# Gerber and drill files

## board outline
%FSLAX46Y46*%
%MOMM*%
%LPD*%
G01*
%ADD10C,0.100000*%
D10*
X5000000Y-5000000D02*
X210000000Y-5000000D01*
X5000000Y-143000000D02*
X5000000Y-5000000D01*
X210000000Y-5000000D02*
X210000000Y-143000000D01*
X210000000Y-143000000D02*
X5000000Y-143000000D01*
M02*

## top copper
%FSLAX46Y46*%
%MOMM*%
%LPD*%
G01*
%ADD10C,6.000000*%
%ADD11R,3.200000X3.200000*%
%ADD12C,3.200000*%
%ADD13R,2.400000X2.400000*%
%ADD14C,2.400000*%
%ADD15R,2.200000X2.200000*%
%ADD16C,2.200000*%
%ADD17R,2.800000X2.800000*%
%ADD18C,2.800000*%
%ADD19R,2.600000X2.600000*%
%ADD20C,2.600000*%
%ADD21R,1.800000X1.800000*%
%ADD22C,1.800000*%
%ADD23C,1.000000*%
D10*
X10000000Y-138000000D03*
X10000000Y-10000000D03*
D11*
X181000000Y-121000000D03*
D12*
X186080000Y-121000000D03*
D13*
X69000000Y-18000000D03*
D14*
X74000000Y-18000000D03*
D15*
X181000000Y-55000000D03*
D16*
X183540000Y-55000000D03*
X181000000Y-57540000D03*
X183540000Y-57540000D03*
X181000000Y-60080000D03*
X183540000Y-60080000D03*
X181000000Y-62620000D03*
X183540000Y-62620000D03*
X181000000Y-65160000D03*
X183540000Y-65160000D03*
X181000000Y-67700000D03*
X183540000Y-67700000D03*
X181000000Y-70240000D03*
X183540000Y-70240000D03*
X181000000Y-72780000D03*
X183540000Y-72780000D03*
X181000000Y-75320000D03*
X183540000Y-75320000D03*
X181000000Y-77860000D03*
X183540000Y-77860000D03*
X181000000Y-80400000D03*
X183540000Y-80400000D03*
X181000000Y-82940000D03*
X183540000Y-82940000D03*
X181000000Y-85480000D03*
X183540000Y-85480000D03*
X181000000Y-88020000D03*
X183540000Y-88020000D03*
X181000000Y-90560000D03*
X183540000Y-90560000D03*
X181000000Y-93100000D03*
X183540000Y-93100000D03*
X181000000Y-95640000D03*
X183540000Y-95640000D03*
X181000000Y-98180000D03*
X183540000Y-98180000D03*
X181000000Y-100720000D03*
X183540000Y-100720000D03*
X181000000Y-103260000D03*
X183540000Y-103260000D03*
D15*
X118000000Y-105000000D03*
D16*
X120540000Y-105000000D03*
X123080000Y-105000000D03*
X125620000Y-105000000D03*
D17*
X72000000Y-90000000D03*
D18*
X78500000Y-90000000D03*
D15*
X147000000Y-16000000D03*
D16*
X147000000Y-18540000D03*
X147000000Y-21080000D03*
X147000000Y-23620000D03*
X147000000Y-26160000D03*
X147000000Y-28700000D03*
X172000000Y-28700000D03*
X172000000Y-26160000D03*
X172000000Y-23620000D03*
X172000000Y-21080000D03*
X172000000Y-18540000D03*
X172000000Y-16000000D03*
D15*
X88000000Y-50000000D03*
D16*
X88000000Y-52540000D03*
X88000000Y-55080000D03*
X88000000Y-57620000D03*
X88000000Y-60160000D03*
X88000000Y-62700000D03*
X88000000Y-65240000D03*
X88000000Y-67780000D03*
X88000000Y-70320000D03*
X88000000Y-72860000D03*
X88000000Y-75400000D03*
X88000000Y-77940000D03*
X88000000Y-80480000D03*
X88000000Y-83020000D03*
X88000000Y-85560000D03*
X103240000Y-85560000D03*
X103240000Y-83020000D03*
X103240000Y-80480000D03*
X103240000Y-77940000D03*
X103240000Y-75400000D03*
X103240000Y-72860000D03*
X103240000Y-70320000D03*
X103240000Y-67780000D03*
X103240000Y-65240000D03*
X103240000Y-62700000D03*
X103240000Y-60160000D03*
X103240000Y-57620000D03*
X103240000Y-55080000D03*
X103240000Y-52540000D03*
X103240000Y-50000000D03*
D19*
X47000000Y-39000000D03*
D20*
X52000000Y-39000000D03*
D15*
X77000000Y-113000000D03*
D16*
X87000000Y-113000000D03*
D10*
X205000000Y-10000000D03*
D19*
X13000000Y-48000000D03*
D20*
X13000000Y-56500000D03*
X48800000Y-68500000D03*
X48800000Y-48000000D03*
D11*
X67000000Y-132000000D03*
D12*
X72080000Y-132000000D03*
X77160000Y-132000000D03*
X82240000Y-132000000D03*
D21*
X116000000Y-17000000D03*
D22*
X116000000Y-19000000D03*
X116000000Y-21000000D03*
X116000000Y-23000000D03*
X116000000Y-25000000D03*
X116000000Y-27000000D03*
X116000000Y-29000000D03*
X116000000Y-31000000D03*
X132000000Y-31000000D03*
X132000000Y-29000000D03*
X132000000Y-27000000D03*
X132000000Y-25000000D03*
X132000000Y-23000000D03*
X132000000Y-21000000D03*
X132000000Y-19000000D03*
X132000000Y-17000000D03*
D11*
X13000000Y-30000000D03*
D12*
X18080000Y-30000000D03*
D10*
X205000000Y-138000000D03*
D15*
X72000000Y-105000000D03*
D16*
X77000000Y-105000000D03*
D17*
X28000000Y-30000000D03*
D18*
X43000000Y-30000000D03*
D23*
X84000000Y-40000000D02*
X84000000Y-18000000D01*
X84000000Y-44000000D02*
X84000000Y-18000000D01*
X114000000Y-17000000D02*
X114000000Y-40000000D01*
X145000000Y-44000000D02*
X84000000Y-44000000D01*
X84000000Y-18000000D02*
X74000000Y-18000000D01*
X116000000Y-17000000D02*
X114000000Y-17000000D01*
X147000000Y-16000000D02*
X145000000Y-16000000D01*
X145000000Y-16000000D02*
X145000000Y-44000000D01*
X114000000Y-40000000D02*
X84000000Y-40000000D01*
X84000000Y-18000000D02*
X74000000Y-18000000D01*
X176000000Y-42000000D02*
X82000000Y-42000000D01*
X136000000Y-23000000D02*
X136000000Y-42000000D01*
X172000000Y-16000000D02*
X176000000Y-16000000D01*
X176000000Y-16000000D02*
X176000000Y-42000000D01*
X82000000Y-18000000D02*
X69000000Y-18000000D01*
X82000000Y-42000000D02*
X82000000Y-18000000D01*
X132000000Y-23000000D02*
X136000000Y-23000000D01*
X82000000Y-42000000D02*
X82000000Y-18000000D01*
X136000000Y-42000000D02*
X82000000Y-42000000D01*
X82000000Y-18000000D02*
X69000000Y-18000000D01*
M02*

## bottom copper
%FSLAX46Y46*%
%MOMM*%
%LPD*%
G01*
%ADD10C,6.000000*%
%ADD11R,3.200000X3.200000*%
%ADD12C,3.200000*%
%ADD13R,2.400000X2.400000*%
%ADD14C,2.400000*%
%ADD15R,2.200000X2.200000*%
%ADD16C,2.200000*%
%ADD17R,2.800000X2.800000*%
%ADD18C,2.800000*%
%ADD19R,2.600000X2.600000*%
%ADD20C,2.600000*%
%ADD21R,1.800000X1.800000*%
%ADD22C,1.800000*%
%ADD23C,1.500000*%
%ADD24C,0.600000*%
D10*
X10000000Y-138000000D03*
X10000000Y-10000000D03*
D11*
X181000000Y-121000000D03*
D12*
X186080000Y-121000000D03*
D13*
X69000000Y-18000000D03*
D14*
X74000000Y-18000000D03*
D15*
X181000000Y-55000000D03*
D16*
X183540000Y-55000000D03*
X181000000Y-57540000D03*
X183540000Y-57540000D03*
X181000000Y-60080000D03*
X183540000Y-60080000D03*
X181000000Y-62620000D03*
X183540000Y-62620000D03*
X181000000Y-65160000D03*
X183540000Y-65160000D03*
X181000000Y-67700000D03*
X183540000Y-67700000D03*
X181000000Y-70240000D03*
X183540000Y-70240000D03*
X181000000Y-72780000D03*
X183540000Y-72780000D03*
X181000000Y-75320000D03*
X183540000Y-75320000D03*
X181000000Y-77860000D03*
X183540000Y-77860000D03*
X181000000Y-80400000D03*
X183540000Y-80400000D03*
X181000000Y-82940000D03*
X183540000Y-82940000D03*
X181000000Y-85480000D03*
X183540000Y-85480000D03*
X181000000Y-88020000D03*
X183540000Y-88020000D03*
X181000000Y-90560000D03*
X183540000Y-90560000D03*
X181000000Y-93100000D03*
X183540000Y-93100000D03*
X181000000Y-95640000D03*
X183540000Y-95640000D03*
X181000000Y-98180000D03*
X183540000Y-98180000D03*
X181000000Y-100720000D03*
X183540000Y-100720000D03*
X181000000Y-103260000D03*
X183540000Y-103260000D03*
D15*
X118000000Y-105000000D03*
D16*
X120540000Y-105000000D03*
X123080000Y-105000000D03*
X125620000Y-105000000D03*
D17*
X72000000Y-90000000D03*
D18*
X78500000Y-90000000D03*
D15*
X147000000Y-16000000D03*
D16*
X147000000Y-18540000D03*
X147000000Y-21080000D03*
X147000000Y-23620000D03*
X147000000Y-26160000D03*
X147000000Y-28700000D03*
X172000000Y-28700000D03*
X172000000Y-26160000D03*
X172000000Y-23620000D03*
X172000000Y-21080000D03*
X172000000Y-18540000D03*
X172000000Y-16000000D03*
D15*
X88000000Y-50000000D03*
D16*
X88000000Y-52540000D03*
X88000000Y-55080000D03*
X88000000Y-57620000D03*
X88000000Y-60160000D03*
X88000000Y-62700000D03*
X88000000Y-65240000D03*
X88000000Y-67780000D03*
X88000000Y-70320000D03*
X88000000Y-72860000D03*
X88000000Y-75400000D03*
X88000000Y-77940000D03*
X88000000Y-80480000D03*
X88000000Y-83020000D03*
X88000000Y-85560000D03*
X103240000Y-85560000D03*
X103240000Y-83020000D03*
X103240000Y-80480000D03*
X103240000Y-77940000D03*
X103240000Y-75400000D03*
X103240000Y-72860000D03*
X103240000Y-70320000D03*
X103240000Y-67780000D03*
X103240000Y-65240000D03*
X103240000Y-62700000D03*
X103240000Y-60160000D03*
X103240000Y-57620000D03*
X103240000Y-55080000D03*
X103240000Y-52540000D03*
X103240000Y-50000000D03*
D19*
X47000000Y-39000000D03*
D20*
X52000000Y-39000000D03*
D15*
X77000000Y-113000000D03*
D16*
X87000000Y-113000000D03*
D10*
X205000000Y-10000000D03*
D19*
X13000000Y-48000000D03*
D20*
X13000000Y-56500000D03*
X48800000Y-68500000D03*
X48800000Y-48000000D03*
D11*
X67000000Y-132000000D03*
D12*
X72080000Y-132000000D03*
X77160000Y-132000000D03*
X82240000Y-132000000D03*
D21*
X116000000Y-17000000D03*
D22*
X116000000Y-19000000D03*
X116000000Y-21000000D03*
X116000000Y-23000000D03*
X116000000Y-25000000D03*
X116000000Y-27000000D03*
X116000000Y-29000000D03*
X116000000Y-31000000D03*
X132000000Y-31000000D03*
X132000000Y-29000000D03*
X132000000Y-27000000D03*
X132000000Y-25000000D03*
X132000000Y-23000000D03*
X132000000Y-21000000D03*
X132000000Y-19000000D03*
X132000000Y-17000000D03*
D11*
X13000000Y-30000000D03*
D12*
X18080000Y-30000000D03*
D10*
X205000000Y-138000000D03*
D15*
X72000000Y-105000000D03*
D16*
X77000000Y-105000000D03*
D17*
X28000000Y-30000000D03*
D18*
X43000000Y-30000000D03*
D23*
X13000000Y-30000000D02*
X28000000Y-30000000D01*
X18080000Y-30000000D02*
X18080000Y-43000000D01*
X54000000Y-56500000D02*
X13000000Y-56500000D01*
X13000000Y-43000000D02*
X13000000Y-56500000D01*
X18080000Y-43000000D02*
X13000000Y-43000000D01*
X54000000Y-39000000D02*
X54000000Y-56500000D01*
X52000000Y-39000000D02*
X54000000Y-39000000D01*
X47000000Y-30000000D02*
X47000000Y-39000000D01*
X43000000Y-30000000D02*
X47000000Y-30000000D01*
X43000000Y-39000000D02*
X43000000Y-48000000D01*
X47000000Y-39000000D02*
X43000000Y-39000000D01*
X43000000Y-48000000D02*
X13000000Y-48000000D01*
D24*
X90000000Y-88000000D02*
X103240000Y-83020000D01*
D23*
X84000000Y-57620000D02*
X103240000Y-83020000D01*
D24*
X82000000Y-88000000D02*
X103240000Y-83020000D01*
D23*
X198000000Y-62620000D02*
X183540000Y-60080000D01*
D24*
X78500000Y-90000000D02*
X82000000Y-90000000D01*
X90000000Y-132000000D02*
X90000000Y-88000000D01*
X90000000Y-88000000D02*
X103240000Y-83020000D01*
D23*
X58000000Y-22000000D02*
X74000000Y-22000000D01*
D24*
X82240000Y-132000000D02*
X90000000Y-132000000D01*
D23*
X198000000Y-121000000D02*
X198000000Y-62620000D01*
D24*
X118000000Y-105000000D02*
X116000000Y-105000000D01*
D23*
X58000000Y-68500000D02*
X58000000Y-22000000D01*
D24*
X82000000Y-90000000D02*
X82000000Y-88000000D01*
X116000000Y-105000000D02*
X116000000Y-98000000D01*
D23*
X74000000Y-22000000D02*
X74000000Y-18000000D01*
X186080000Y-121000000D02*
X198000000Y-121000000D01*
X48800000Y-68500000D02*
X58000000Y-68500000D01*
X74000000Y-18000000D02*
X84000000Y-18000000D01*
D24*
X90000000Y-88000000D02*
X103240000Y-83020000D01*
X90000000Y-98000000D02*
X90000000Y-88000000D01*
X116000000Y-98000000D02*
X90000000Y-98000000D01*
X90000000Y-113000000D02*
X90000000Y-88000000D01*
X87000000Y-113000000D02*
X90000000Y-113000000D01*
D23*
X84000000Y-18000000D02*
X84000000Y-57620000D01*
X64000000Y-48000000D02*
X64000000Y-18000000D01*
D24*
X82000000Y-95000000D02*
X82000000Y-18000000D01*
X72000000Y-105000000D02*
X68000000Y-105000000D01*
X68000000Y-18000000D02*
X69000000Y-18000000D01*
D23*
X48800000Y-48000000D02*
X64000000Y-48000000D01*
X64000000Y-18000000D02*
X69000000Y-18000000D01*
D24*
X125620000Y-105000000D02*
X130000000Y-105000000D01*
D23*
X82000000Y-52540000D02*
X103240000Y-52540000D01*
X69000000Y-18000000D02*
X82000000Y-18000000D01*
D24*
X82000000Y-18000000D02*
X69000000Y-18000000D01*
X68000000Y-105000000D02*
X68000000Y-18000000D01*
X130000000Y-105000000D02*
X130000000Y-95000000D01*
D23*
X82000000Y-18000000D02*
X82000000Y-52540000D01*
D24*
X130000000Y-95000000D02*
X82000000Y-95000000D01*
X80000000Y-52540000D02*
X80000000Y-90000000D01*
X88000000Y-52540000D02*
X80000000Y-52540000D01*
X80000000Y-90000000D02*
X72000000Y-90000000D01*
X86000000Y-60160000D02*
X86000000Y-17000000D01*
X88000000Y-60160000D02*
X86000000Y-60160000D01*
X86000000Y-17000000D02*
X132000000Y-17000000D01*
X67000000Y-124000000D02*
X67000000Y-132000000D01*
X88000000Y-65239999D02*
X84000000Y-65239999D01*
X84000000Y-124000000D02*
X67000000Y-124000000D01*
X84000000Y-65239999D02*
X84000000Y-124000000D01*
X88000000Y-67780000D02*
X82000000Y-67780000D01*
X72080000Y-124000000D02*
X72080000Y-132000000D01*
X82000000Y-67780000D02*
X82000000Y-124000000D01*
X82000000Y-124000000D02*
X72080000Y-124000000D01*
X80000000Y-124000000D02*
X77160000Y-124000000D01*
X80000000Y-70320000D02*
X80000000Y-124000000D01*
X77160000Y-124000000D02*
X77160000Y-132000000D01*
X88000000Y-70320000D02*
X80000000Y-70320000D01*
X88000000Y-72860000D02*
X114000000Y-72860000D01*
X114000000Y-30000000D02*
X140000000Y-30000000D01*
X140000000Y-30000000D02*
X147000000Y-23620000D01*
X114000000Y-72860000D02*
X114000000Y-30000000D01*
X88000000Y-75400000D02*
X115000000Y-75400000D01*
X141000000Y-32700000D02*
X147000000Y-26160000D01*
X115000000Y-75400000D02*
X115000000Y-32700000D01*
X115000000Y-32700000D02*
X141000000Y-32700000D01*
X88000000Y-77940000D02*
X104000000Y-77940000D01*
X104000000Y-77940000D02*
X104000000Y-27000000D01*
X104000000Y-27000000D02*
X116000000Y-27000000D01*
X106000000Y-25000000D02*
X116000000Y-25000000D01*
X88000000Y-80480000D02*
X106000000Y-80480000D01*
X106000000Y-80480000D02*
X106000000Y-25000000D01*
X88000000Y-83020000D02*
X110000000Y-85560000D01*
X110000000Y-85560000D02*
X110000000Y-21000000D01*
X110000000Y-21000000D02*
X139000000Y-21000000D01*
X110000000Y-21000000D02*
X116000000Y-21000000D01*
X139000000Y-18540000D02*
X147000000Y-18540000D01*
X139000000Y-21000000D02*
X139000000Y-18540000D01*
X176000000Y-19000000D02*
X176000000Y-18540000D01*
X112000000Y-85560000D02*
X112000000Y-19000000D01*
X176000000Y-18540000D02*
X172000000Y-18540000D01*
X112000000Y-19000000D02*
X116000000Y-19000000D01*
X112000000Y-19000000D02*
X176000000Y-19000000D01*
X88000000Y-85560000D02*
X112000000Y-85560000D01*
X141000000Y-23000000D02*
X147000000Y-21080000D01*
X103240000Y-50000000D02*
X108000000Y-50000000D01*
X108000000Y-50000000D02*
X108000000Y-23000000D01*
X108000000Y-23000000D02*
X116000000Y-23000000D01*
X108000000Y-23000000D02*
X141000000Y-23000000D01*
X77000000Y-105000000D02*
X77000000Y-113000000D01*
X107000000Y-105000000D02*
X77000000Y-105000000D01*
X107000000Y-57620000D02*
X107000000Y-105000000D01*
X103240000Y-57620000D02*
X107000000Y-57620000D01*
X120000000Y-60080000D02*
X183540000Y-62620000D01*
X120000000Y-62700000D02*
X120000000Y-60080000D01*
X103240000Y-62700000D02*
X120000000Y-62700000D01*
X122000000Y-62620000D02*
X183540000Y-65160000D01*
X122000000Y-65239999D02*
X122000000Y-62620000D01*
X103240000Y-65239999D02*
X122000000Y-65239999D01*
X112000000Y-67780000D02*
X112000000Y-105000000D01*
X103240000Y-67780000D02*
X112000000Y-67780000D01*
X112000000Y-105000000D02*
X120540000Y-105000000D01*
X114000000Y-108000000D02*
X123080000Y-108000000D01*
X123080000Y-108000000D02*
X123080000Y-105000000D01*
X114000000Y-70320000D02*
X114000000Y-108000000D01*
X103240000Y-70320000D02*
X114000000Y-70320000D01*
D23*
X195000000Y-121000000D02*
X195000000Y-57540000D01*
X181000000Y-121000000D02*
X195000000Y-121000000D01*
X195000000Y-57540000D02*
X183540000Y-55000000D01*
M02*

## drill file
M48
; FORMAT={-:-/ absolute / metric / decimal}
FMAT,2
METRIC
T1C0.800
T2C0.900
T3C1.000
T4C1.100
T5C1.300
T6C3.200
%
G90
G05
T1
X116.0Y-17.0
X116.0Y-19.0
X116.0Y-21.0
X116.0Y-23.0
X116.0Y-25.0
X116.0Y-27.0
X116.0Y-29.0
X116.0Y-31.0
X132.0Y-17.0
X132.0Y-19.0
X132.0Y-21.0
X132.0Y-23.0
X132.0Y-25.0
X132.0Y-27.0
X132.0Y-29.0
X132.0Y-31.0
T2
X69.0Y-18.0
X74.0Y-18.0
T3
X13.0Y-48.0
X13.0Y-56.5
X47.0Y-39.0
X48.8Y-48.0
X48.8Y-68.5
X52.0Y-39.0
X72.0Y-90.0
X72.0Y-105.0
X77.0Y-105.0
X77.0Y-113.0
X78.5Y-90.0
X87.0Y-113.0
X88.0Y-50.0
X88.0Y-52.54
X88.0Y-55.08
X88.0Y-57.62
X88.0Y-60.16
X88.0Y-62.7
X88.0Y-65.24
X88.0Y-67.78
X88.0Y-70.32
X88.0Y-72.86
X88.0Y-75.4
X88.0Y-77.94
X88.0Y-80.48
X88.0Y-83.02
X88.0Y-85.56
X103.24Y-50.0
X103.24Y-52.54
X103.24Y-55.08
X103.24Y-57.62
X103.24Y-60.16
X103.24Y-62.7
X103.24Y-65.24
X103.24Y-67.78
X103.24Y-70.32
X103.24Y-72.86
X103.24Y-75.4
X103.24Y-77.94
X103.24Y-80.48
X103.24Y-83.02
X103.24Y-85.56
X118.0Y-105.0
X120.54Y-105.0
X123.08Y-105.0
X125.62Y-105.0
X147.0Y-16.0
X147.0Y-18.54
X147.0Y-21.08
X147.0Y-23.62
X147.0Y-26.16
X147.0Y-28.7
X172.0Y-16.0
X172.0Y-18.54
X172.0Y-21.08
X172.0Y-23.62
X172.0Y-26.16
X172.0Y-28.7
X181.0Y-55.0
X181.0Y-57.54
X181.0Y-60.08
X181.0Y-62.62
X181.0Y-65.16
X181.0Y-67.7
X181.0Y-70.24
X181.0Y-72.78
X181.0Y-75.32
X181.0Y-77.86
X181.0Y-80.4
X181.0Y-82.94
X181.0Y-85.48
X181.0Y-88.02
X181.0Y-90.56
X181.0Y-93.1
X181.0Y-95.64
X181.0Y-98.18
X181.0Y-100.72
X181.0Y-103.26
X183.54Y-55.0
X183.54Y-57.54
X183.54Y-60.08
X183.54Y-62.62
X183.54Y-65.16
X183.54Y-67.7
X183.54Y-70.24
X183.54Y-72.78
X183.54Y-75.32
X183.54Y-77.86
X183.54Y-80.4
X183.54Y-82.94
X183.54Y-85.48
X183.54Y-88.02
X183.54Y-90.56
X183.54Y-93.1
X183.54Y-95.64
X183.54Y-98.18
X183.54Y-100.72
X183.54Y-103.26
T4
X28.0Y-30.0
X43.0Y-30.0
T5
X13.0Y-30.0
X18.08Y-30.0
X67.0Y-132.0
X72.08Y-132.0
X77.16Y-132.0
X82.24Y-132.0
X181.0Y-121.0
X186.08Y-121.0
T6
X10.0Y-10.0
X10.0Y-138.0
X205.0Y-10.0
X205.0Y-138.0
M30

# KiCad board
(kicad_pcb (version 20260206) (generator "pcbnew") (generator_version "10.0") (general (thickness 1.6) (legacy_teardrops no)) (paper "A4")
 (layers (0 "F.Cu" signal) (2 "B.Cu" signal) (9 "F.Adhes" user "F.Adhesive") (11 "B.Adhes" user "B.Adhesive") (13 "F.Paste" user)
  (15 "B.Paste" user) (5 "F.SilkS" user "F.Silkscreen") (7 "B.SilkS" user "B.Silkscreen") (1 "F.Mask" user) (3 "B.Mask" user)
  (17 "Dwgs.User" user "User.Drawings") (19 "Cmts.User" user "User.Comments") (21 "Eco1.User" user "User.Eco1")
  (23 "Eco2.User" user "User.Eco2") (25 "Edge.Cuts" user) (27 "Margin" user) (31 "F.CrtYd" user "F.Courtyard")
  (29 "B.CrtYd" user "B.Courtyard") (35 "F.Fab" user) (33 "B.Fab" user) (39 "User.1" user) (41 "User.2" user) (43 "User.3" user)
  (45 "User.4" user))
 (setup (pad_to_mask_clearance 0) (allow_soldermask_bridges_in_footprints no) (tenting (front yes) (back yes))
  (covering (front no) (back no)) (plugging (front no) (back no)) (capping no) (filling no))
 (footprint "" (layer "F.Cu") (at 10 138)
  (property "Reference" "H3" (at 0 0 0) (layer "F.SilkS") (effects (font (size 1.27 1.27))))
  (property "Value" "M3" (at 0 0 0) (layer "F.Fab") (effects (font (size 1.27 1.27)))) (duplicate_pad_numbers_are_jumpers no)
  (pad "1" thru_hole circle (at 0 0) (size 6 6) (drill 3.2) (layers "*.Cu" "*.Mask") (remove_unused_layers no)))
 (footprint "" (layer "F.Cu") (at 10 10)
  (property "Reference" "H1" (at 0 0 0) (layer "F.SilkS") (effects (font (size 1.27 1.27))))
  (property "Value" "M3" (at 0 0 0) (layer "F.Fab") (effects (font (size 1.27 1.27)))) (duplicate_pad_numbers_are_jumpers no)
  (pad "1" thru_hole circle (at 0 0) (size 6 6) (drill 3.2) (layers "*.Cu" "*.Mask") (remove_unused_layers no)))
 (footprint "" (layer "F.Cu") (at 181 121)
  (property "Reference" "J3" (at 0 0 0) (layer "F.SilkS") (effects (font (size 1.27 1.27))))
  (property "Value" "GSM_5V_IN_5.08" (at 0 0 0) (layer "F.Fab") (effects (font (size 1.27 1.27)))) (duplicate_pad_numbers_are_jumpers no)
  (pad "1" thru_hole rect (at 0 0) (size 3.2 3.2) (drill 1.3) (layers "*.Cu" "*.Mask") (remove_unused_layers no) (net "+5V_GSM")
   (thermal_bridge_angle 45))
  (pad "2" thru_hole circle (at 5.08 0) (size 3.2 3.2) (drill 1.3) (layers "*.Cu" "*.Mask") (remove_unused_layers no) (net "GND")))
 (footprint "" (layer "F.Cu") (at 69 18)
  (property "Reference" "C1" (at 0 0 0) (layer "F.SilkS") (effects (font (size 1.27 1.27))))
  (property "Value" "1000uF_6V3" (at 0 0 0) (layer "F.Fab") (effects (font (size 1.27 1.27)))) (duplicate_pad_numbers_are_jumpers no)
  (pad "1" thru_hole rect (at 0 0) (size 2.4 2.4) (drill 0.9) (layers "*.Cu" "*.Mask") (remove_unused_layers no) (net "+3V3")
   (thermal_bridge_angle 45))
  (pad "2" thru_hole circle (at 5 0) (size 2.4 2.4) (drill 0.9) (layers "*.Cu" "*.Mask") (remove_unused_layers no) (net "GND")))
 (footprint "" (layer "F.Cu") (at 181 55)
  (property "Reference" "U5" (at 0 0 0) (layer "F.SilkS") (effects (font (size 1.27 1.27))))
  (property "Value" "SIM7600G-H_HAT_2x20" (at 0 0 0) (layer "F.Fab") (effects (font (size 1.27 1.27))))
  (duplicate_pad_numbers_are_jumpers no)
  (pad "1" thru_hole rect (at 0 0) (size 2.2 2.2) (drill 1) (layers "*.Cu" "*.Mask") (remove_unused_layers no) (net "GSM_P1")
   (thermal_bridge_angle 45))
  (pad "2" thru_hole circle (at 2.54 0) (size 2.2 2.2) (drill 1) (layers "*.Cu" "*.Mask") (remove_unused_layers no) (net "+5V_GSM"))
  (pad "3" thru_hole circle (at 0 2.54) (size 2.2 2.2) (drill 1) (layers "*.Cu" "*.Mask") (remove_unused_layers no) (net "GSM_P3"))
  (pad "4" thru_hole circle (at 2.54 2.54) (size 2.2 2.2) (drill 1) (layers "*.Cu" "*.Mask") (remove_unused_layers no) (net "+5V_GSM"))
  (pad "5" thru_hole circle (at 0 5.08) (size 2.2 2.2) (drill 1) (layers "*.Cu" "*.Mask") (remove_unused_layers no) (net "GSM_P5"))
  (pad "6" thru_hole circle (at 2.54 5.08) (size 2.2 2.2) (drill 1) (layers "*.Cu" "*.Mask") (remove_unused_layers no) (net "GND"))
  (pad "7" thru_hole circle (at 0 7.62) (size 2.2 2.2) (drill 1) (layers "*.Cu" "*.Mask") (remove_unused_layers no) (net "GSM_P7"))
  (pad "8" thru_hole circle (at 2.54 7.62) (size 2.2 2.2) (drill 1) (layers "*.Cu" "*.Mask") (remove_unused_layers no) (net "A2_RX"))
  (pad "9" thru_hole circle (at 0 10.16) (size 2.2 2.2) (drill 1) (layers "*.Cu" "*.Mask") (remove_unused_layers no) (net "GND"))
  (pad "10" thru_hole circle (at 2.54 10.16) (size 2.2 2.2) (drill 1) (layers "*.Cu" "*.Mask") (remove_unused_layers no) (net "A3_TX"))
  (pad "11" thru_hole circle (at 0 12.7) (size 2.2 2.2) (drill 1) (layers "*.Cu" "*.Mask") (remove_unused_layers no) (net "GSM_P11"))
  (pad "12" thru_hole circle (at 2.54 12.7) (size 2.2 2.2) (drill 1) (layers "*.Cu" "*.Mask") (remove_unused_layers no) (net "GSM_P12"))
  (pad "13" thru_hole circle (at 0 15.24) (size 2.2 2.2) (drill 1) (layers "*.Cu" "*.Mask") (remove_unused_layers no) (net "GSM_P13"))
  (pad "14" thru_hole circle (at 2.54 15.24) (size 2.2 2.2) (drill 1) (layers "*.Cu" "*.Mask") (remove_unused_layers no) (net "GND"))
  (pad "15" thru_hole circle (at 0 17.78) (size 2.2 2.2) (drill 1) (layers "*.Cu" "*.Mask") (remove_unused_layers no) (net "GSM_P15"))
  (pad "16" thru_hole circle (at 2.54 17.78) (size 2.2 2.2) (drill 1) (layers "*.Cu" "*.Mask") (remove_unused_layers no) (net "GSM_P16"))
  (pad "17" thru_hole circle (at 0 20.32) (size 2.2 2.2) (drill 1) (layers "*.Cu" "*.Mask") (remove_unused_layers no) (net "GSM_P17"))
  (pad "18" thru_hole circle (at 2.54 20.32) (size 2.2 2.2) (drill 1) (layers "*.Cu" "*.Mask") (remove_unused_layers no) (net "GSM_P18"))
  (pad "19" thru_hole circle (at 0 22.86) (size 2.2 2.2) (drill 1) (layers "*.Cu" "*.Mask") (remove_unused_layers no) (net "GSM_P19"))
  (pad "20" thru_hole circle (at 2.54 22.86) (size 2.2 2.2) (drill 1) (layers "*.Cu" "*.Mask") (remove_unused_layers no) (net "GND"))
  (pad "21" thru_hole circle (at 0 25.4) (size 2.2 2.2) (drill 1) (layers "*.Cu" "*.Mask") (remove_unused_layers no) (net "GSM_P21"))
  (pad "22" thru_hole circle (at 2.54 25.4) (size 2.2 2.2) (drill 1) (layers "*.Cu" "*.Mask") (remove_unused_layers no) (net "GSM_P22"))
  (pad "23" thru_hole circle (at 0 27.94) (size 2.2 2.2) (drill 1) (layers "*.Cu" "*.Mask") (remove_unused_layers no) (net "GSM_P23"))
  (pad "24" thru_hole circle (at 2.54 27.94) (size 2.2 2.2) (drill 1) (layers "*.Cu" "*.Mask") (remove_unused_layers no) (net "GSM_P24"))
  (pad "25" thru_hole circle (at 0 30.48) (size 2.2 2.2) (drill 1) (layers "*.Cu" "*.Mask") (remove_unused_layers no) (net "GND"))
  (pad "26" thru_hole circle (at 2.54 30.48) (size 2.2 2.2) (drill 1) (layers "*.Cu" "*.Mask") (remove_unused_layers no) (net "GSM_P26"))
  (pad "27" thru_hole circle (at 0 33.02) (size 2.2 2.2) (drill 1) (layers "*.Cu" "*.Mask") (remove_unused_layers no) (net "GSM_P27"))
  (pad "28" thru_hole circle (at 2.54 33.02) (size 2.2 2.2) (drill 1) (layers "*.Cu" "*.Mask") (remove_unused_layers no) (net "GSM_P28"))
  (pad "29" thru_hole circle (at 0 35.56) (size 2.2 2.2) (drill 1) (layers "*.Cu" "*.Mask") (remove_unused_layers no) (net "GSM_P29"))
  (pad "30" thru_hole circle (at 2.54 35.56) (size 2.2 2.2) (drill 1) (layers "*.Cu" "*.Mask") (remove_unused_layers no) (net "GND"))
  (pad "31" thru_hole circle (at 0 38.1) (size 2.2 2.2) (drill 1) (layers "*.Cu" "*.Mask") (remove_unused_layers no) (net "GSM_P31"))
  (pad "32" thru_hole circle (at 2.54 38.1) (size 2.2 2.2) (drill 1) (layers "*.Cu" "*.Mask") (remove_unused_layers no) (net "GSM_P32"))
  (pad "33" thru_hole circle (at 0 40.64) (size 2.2 2.2) (drill 1) (layers "*.Cu" "*.Mask") (remove_unused_layers no) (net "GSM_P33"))
  (pad "34" thru_hole circle (at 2.54 40.64) (size 2.2 2.2) (drill 1) (layers "*.Cu" "*.Mask") (remove_unused_layers no) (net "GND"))
  (pad "35" thru_hole circle (at 0 43.18) (size 2.2 2.2) (drill 1) (layers "*.Cu" "*.Mask") (remove_unused_layers no) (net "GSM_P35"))
  (pad "36" thru_hole circle (at 2.54 43.18) (size 2.2 2.2) (drill 1) (layers "*.Cu" "*.Mask") (remove_unused_layers no) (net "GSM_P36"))
  (pad "37" thru_hole circle (at 0 45.72) (size 2.2 2.2) (drill 1) (layers "*.Cu" "*.Mask") (remove_unused_layers no) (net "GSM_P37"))
  (pad "38" thru_hole circle (at 2.54 45.72) (size 2.2 2.2) (drill 1) (layers "*.Cu" "*.Mask") (remove_unused_layers no) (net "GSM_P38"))
  (pad "39" thru_hole circle (at 0 48.26) (size 2.2 2.2) (drill 1) (layers "*.Cu" "*.Mask") (remove_unused_layers no) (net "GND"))
  (pad "40" thru_hole circle (at 2.54 48.26) (size 2.2 2.2) (drill 1) (layers "*.Cu" "*.Mask") (remove_unused_layers no) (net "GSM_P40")))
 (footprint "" (layer "F.Cu") (at 118 105)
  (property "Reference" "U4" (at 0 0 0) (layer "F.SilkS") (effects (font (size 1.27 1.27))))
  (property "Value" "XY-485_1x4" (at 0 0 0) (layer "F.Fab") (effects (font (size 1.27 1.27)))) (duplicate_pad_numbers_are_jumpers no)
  (pad "1" thru_hole rect (at 0 0) (size 2.2 2.2) (drill 1) (layers "*.Cu" "*.Mask") (remove_unused_layers no) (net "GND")
   (thermal_bridge_angle 45))
  (pad "2" thru_hole circle (at 2.54 0) (size 2.2 2.2) (drill 1) (layers "*.Cu" "*.Mask") (remove_unused_layers no) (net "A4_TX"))
  (pad "3" thru_hole circle (at 5.08 0) (size 2.2 2.2) (drill 1) (layers "*.Cu" "*.Mask") (remove_unused_layers no) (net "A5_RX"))
  (pad "4" thru_hole circle (at 7.62 0) (size 2.2 2.2) (drill 1) (layers "*.Cu" "*.Mask") (remove_unused_layers no) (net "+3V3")))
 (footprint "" (layer "F.Cu") (at 72 90)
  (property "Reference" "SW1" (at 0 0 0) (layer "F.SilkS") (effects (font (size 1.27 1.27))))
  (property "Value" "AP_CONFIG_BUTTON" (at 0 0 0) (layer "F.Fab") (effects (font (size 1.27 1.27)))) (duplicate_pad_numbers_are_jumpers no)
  (pad "1" thru_hole rect (at 0 0) (size 2.8 2.8) (drill 1) (layers "*.Cu" "*.Mask") (remove_unused_layers no) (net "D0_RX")
   (thermal_bridge_angle 45))
  (pad "2" thru_hole circle (at 6.5 0) (size 2.8 2.8) (drill 1) (layers "*.Cu" "*.Mask") (remove_unused_layers no) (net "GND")))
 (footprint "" (layer "F.Cu") (at 147 16)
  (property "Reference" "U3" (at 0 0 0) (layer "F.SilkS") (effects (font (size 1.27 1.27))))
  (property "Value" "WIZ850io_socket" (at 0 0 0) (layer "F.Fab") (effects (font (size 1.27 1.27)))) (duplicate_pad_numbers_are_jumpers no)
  (pad "1" thru_hole rect (at 0 0) (size 2.2 2.2) (drill 1) (layers "*.Cu" "*.Mask") (remove_unused_layers no) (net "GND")
   (thermal_bridge_angle 45))
  (pad "2" thru_hole circle (at 0 2.54) (size 2.2 2.2) (drill 1) (layers "*.Cu" "*.Mask") (remove_unused_layers no) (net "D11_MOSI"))
  (pad "3" thru_hole circle (at 0 5.08) (size 2.2 2.2) (drill 1) (layers "*.Cu" "*.Mask") (remove_unused_layers no) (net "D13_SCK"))
  (pad "4" thru_hole circle (at 0 7.62) (size 2.2 2.2) (drill 1) (layers "*.Cu" "*.Mask") (remove_unused_layers no) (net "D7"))
  (pad "5" thru_hole circle (at 0 10.16) (size 2.2 2.2) (drill 1) (layers "*.Cu" "*.Mask") (remove_unused_layers no) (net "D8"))
  (pad "6" thru_hole circle (at 0 12.7) (size 2.2 2.2) (drill 1) (layers "*.Cu" "*.Mask") (remove_unused_layers no) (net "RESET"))
  (pad "7" thru_hole circle (at 25 12.7) (size 2.2 2.2) (drill 1) (layers "*.Cu" "*.Mask") (remove_unused_layers no) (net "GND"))
  (pad "8" thru_hole circle (at 25 10.16) (size 2.2 2.2) (drill 1) (layers "*.Cu" "*.Mask") (remove_unused_layers no) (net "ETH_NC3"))
  (pad "9" thru_hole circle (at 25 7.62) (size 2.2 2.2) (drill 1) (layers "*.Cu" "*.Mask") (remove_unused_layers no) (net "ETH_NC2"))
  (pad "10" thru_hole circle (at 25 5.08) (size 2.2 2.2) (drill 1) (layers "*.Cu" "*.Mask") (remove_unused_layers no) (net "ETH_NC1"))
  (pad "11" thru_hole circle (at 25 2.54) (size 2.2 2.2) (drill 1) (layers "*.Cu" "*.Mask") (remove_unused_layers no) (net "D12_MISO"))
  (pad "12" thru_hole circle (at 25 0) (size 2.2 2.2) (drill 1) (layers "*.Cu" "*.Mask") (remove_unused_layers no) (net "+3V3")))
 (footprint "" (layer "F.Cu") (at 88 50)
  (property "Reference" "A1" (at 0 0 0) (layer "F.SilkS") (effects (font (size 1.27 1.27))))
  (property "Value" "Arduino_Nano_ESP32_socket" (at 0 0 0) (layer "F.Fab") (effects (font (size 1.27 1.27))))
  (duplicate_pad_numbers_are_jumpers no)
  (pad "1" thru_hole rect (at 0 0) (size 2.2 2.2) (drill 1) (layers "*.Cu" "*.Mask") (remove_unused_layers no) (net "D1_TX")
   (thermal_bridge_angle 45))
  (pad "2" thru_hole circle (at 0 2.54) (size 2.2 2.2) (drill 1) (layers "*.Cu" "*.Mask") (remove_unused_layers no) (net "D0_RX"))
  (pad "3" thru_hole circle (at 0 5.08) (size 2.2 2.2) (drill 1) (layers "*.Cu" "*.Mask") (remove_unused_layers no) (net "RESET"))
  (pad "4" thru_hole circle (at 0 7.62) (size 2.2 2.2) (drill 1) (layers "*.Cu" "*.Mask") (remove_unused_layers no) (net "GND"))
  (pad "5" thru_hole circle (at 0 10.16) (size 2.2 2.2) (drill 1) (layers "*.Cu" "*.Mask") (remove_unused_layers no) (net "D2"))
  (pad "6" thru_hole circle (at 0 12.7) (size 2.2 2.2) (drill 1) (layers "*.Cu" "*.Mask") (remove_unused_layers no) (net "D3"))
  (pad "7" thru_hole circle (at 0 15.24) (size 2.2 2.2) (drill 1) (layers "*.Cu" "*.Mask") (remove_unused_layers no) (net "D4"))
  (pad "8" thru_hole circle (at 0 17.78) (size 2.2 2.2) (drill 1) (layers "*.Cu" "*.Mask") (remove_unused_layers no) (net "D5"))
  (pad "9" thru_hole circle (at 0 20.32) (size 2.2 2.2) (drill 1) (layers "*.Cu" "*.Mask") (remove_unused_layers no) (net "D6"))
  (pad "10" thru_hole circle (at 0 22.86) (size 2.2 2.2) (drill 1) (layers "*.Cu" "*.Mask") (remove_unused_layers no) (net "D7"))
  (pad "11" thru_hole circle (at 0 25.4) (size 2.2 2.2) (drill 1) (layers "*.Cu" "*.Mask") (remove_unused_layers no) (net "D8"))
  (pad "12" thru_hole circle (at 0 27.94) (size 2.2 2.2) (drill 1) (layers "*.Cu" "*.Mask") (remove_unused_layers no) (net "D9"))
  (pad "13" thru_hole circle (at 0 30.48) (size 2.2 2.2) (drill 1) (layers "*.Cu" "*.Mask") (remove_unused_layers no) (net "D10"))
  (pad "14" thru_hole circle (at 0 33.02) (size 2.2 2.2) (drill 1) (layers "*.Cu" "*.Mask") (remove_unused_layers no) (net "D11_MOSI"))
  (pad "15" thru_hole circle (at 0 35.56) (size 2.2 2.2) (drill 1) (layers "*.Cu" "*.Mask") (remove_unused_layers no) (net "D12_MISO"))
  (pad "16" thru_hole circle (at 15.24 35.56) (size 2.2 2.2) (drill 1) (layers "*.Cu" "*.Mask") (remove_unused_layers no) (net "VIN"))
  (pad "17" thru_hole circle (at 15.24 33.02) (size 2.2 2.2) (drill 1) (layers "*.Cu" "*.Mask") (remove_unused_layers no) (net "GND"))
  (pad "18" thru_hole circle (at 15.24 30.48) (size 2.2 2.2) (drill 1) (layers "*.Cu" "*.Mask") (remove_unused_layers no) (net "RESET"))
  (pad "19" thru_hole circle (at 15.24 27.94) (size 2.2 2.2) (drill 1) (layers "*.Cu" "*.Mask") (remove_unused_layers no) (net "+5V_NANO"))
  (pad "20" thru_hole circle (at 15.24 25.4) (size 2.2 2.2) (drill 1) (layers "*.Cu" "*.Mask") (remove_unused_layers no) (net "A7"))
  (pad "21" thru_hole circle (at 15.24 22.86) (size 2.2 2.2) (drill 1) (layers "*.Cu" "*.Mask") (remove_unused_layers no) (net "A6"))
  (pad "22" thru_hole circle (at 15.24 20.32) (size 2.2 2.2) (drill 1) (layers "*.Cu" "*.Mask") (remove_unused_layers no) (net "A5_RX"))
  (pad "23" thru_hole circle (at 15.24 17.78) (size 2.2 2.2) (drill 1) (layers "*.Cu" "*.Mask") (remove_unused_layers no) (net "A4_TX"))
  (pad "24" thru_hole circle (at 15.24 15.24) (size 2.2 2.2) (drill 1) (layers "*.Cu" "*.Mask") (remove_unused_layers no) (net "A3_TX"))
  (pad "25" thru_hole circle (at 15.24 12.7) (size 2.2 2.2) (drill 1) (layers "*.Cu" "*.Mask") (remove_unused_layers no) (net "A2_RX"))
  (pad "26" thru_hole circle (at 15.24 10.16) (size 2.2 2.2) (drill 1) (layers "*.Cu" "*.Mask") (remove_unused_layers no) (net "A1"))
  (pad "27" thru_hole circle (at 15.24 7.62) (size 2.2 2.2) (drill 1) (layers "*.Cu" "*.Mask") (remove_unused_layers no) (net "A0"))
  (pad "28" thru_hole circle (at 15.24 5.08) (size 2.2 2.2) (drill 1) (layers "*.Cu" "*.Mask") (remove_unused_layers no) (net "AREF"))
  (pad "29" thru_hole circle (at 15.24 2.54) (size 2.2 2.2) (drill 1) (layers "*.Cu" "*.Mask") (remove_unused_layers no) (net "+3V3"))
  (pad "30" thru_hole circle (at 15.24 0) (size 2.2 2.2) (drill 1) (layers "*.Cu" "*.Mask") (remove_unused_layers no) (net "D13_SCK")))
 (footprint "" (layer "F.Cu") (at 47 39)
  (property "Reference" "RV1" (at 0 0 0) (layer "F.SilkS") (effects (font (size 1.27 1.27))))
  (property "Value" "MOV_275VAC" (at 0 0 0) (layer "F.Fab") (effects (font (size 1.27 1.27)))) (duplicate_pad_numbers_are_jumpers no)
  (pad "1" thru_hole rect (at 0 0) (size 2.6 2.6) (drill 1) (layers "*.Cu" "*.Mask") (remove_unused_layers no) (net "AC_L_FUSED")
   (thermal_bridge_angle 45))
  (pad "2" thru_hole circle (at 5 0) (size 2.6 2.6) (drill 1) (layers "*.Cu" "*.Mask") (remove_unused_layers no) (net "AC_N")))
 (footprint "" (layer "F.Cu") (at 77 113)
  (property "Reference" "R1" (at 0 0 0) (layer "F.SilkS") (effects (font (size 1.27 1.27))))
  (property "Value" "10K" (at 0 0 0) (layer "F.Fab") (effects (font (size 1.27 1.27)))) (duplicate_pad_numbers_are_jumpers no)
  (pad "1" thru_hole rect (at 0 0) (size 2.2 2.2) (drill 1) (layers "*.Cu" "*.Mask") (remove_unused_layers no) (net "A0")
   (thermal_bridge_angle 45))
  (pad "2" thru_hole circle (at 10 0) (size 2.2 2.2) (drill 1) (layers "*.Cu" "*.Mask") (remove_unused_layers no) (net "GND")))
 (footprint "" (layer "F.Cu") (at 205 10)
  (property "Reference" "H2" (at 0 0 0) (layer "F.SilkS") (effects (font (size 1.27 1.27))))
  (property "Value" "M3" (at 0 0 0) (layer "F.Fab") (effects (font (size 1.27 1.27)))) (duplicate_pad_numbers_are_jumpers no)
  (pad "1" thru_hole circle (at 0 0) (size 6 6) (drill 3.2) (layers "*.Cu" "*.Mask") (remove_unused_layers no)))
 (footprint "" (layer "F.Cu") (at 13 48)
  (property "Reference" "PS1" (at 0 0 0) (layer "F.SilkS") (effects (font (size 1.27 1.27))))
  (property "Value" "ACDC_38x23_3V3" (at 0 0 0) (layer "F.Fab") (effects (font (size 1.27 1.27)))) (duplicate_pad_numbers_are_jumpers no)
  (pad "1" thru_hole rect (at 0 0) (size 2.6 2.6) (drill 1) (layers "*.Cu" "*.Mask") (remove_unused_layers no) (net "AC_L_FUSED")
   (thermal_bridge_angle 45))
  (pad "2" thru_hole circle (at 0 8.5) (size 2.6 2.6) (drill 1) (layers "*.Cu" "*.Mask") (remove_unused_layers no) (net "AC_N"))
  (pad "3" thru_hole circle (at 35.8 20.5) (size 2.6 2.6) (drill 1) (layers "*.Cu" "*.Mask") (remove_unused_layers no) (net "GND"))
  (pad "4" thru_hole circle (at 35.8 0) (size 2.6 2.6) (drill 1) (layers "*.Cu" "*.Mask") (remove_unused_layers no) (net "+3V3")))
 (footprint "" (layer "F.Cu") (at 67 132)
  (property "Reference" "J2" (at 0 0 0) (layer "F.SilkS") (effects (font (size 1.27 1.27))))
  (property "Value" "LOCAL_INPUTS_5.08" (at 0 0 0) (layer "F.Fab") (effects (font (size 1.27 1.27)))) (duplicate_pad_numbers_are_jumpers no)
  (pad "1" thru_hole rect (at 0 0) (size 3.2 3.2) (drill 1.3) (layers "*.Cu" "*.Mask") (remove_unused_layers no) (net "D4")
   (thermal_bridge_angle 45))
  (pad "2" thru_hole circle (at 5.08 0) (size 3.2 3.2) (drill 1.3) (layers "*.Cu" "*.Mask") (remove_unused_layers no) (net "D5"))
  (pad "3" thru_hole circle (at 10.16 0) (size 3.2 3.2) (drill 1.3) (layers "*.Cu" "*.Mask") (remove_unused_layers no) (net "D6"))
  (pad "4" thru_hole circle (at 15.24 0) (size 3.2 3.2) (drill 1.3) (layers "*.Cu" "*.Mask") (remove_unused_layers no) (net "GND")))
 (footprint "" (layer "F.Cu") (at 116 17)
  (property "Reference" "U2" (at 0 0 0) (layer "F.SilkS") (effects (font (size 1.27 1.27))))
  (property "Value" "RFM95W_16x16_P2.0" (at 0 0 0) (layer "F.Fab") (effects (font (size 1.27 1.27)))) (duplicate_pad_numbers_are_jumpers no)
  (pad "1" thru_hole rect (at 0 0) (size 1.8 1.8) (drill 0.8) (layers "*.Cu" "*.Mask") (remove_unused_layers no) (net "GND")
   (thermal_bridge_angle 45))
  (pad "2" thru_hole circle (at 0 2) (size 1.8 1.8) (drill 0.8) (layers "*.Cu" "*.Mask") (remove_unused_layers no) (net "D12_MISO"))
  (pad "3" thru_hole circle (at 0 4) (size 1.8 1.8) (drill 0.8) (layers "*.Cu" "*.Mask") (remove_unused_layers no) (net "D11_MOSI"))
  (pad "4" thru_hole circle (at 0 6) (size 1.8 1.8) (drill 0.8) (layers "*.Cu" "*.Mask") (remove_unused_layers no) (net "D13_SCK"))
  (pad "5" thru_hole circle (at 0 8) (size 1.8 1.8) (drill 0.8) (layers "*.Cu" "*.Mask") (remove_unused_layers no) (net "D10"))
  (pad "6" thru_hole circle (at 0 10) (size 1.8 1.8) (drill 0.8) (layers "*.Cu" "*.Mask") (remove_unused_layers no) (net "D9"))
  (pad "7" thru_hole circle (at 0 12) (size 1.8 1.8) (drill 0.8) (layers "*.Cu" "*.Mask") (remove_unused_layers no) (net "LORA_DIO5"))
  (pad "8" thru_hole circle (at 0 14) (size 1.8 1.8) (drill 0.8) (layers "*.Cu" "*.Mask") (remove_unused_layers no) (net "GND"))
  (pad "9" thru_hole circle (at 16 14) (size 1.8 1.8) (drill 0.8) (layers "*.Cu" "*.Mask") (remove_unused_layers no) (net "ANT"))
  (pad "10" thru_hole circle (at 16 12) (size 1.8 1.8) (drill 0.8) (layers "*.Cu" "*.Mask") (remove_unused_layers no) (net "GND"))
  (pad "11" thru_hole circle (at 16 10) (size 1.8 1.8) (drill 0.8) (layers "*.Cu" "*.Mask") (remove_unused_layers no) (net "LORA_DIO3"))
  (pad "12" thru_hole circle (at 16 8) (size 1.8 1.8) (drill 0.8) (layers "*.Cu" "*.Mask") (remove_unused_layers no) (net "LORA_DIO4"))
  (pad "13" thru_hole circle (at 16 6) (size 1.8 1.8) (drill 0.8) (layers "*.Cu" "*.Mask") (remove_unused_layers no) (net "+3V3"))
  (pad "14" thru_hole circle (at 16 4) (size 1.8 1.8) (drill 0.8) (layers "*.Cu" "*.Mask") (remove_unused_layers no) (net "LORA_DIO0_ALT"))
  (pad "15" thru_hole circle (at 16 2) (size 1.8 1.8) (drill 0.8) (layers "*.Cu" "*.Mask") (remove_unused_layers no) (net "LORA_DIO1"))
  (pad "16" thru_hole circle (at 16 0) (size 1.8 1.8) (drill 0.8) (layers "*.Cu" "*.Mask") (remove_unused_layers no) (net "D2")))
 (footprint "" (layer "F.Cu") (at 13 30)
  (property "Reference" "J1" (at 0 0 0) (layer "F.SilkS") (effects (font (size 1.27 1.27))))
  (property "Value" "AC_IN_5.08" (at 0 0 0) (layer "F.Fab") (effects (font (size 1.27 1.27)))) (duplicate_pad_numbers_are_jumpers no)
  (pad "1" thru_hole rect (at 0 0) (size 3.2 3.2) (drill 1.3) (layers "*.Cu" "*.Mask") (remove_unused_layers no) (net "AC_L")
   (thermal_bridge_angle 45))
  (pad "2" thru_hole circle (at 5.08 0) (size 3.2 3.2) (drill 1.3) (layers "*.Cu" "*.Mask") (remove_unused_layers no) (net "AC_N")))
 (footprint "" (layer "F.Cu") (at 205 138)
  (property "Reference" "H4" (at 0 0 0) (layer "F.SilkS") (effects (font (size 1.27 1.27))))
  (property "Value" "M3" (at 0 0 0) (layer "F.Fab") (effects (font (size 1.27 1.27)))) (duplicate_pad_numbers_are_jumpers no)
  (pad "1" thru_hole circle (at 0 0) (size 6 6) (drill 3.2) (layers "*.Cu" "*.Mask") (remove_unused_layers no)))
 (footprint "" (layer "F.Cu") (at 72 105)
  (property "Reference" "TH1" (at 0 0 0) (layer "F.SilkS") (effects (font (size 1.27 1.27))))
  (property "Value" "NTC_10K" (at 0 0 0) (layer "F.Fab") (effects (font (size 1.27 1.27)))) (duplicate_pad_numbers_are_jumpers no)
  (pad "1" thru_hole rect (at 0 0) (size 2.2 2.2) (drill 1) (layers "*.Cu" "*.Mask") (remove_unused_layers no) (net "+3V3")
   (thermal_bridge_angle 45))
  (pad "2" thru_hole circle (at 5 0) (size 2.2 2.2) (drill 1) (layers "*.Cu" "*.Mask") (remove_unused_layers no) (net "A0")))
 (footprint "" (layer "F.Cu") (at 28 30)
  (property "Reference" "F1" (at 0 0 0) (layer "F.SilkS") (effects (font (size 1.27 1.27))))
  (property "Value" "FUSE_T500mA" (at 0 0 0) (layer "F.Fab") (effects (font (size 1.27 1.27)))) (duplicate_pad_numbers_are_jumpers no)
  (pad "1" thru_hole rect (at 0 0) (size 2.8 2.8) (drill 1.1) (layers "*.Cu" "*.Mask") (remove_unused_layers no) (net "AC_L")
   (thermal_bridge_angle 45))
  (pad "2" thru_hole circle (at 15 0) (size 2.8 2.8) (drill 1.1) (layers "*.Cu" "*.Mask") (remove_unused_layers no) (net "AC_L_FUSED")))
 (gr_line (start 5 5) (end 210 5) (stroke (width 0.1) (type default)) (layer "Edge.Cuts"))
 (gr_line (start 5 143) (end 5 5) (stroke (width 0.1) (type default)) (layer "Edge.Cuts"))
 (gr_line (start 210 5) (end 210 143) (stroke (width 0.1) (type default)) (layer "Edge.Cuts"))
 (gr_line (start 210 143) (end 5 143) (stroke (width 0.1) (type default)) (layer "Edge.Cuts"))
 (segment (start 13 30) (end 28 30) (width 1.5) (layer "B.Cu") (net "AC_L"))
 (segment (start 18.08 30) (end 18.08 43) (width 1.5) (layer "B.Cu") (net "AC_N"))
 (segment (start 54 56.5) (end 13 56.5) (width 1.5) (layer "B.Cu") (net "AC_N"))
 (segment (start 13 43) (end 13 56.5) (width 1.5) (layer "B.Cu") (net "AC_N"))
 (segment (start 18.08 43) (end 13 43) (width 1.5) (layer "B.Cu") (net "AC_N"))
 (segment (start 54 39) (end 54 56.5) (width 1.5) (layer "B.Cu") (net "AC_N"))
 (segment (start 52 39) (end 54 39) (width 1.5) (layer "B.Cu") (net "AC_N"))
 (segment (start 47 30) (end 47 39) (width 1.5) (layer "B.Cu") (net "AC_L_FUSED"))
 (segment (start 43 30) (end 47 30) (width 1.5) (layer "B.Cu") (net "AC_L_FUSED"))
 (segment (start 43 39) (end 43 48) (width 1.5) (layer "B.Cu") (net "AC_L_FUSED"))
 (segment (start 47 39) (end 43 39) (width 1.5) (layer "B.Cu") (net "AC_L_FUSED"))
 (segment (start 43 48) (end 13 48) (width 1.5) (layer "B.Cu") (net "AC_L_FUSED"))
 (segment (start 84 40) (end 84 18) (width 1) (layer "F.Cu") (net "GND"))
 (segment (start 84 44) (end 84 18) (width 1) (layer "F.Cu") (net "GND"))
 (segment (start 114 17) (end 114 40) (width 1) (layer "F.Cu") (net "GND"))
 (segment (start 145 44) (end 84 44) (width 1) (layer "F.Cu") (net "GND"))
 (segment (start 84 18) (end 74 18) (width 1) (layer "F.Cu") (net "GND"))
 (segment (start 116 17) (end 114 17) (width 1) (layer "F.Cu") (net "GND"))
 (segment (start 147 16) (end 145 16) (width 1) (layer "F.Cu") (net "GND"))
 (segment (start 145 16) (end 145 44) (width 1) (layer "F.Cu") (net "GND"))
 (segment (start 114 40) (end 84 40) (width 1) (layer "F.Cu") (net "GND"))
 (segment (start 84 18) (end 74 18) (width 1) (layer "F.Cu") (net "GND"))
 (segment (start 90 88) (end 103.24 83.02) (width 0.6) (layer "B.Cu") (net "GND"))
 (segment (start 84 57.62) (end 103.24 83.02) (width 1.5) (layer "B.Cu") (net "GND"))
 (segment (start 82 88) (end 103.24 83.02) (width 0.6) (layer "B.Cu") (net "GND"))
 (segment (start 198 62.62) (end 183.54 60.08) (width 1.5) (layer "B.Cu") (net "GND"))
 (segment (start 78.5 90) (end 82 90) (width 0.6) (layer "B.Cu") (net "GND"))
 (segment (start 90 132) (end 90 88) (width 0.6) (layer "B.Cu") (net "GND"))
 (segment (start 90 88) (end 103.24 83.02) (width 0.6) (layer "B.Cu") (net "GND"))
 (segment (start 58 22) (end 74 22) (width 1.5) (layer "B.Cu") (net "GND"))
 (segment (start 82.24 132) (end 90 132) (width 0.6) (layer "B.Cu") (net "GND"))
 (segment (start 198 121) (end 198 62.62) (width 1.5) (layer "B.Cu") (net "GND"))
 (segment (start 118 105) (end 116 105) (width 0.6) (layer "B.Cu") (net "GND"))
 (segment (start 58 68.5) (end 58 22) (width 1.5) (layer "B.Cu") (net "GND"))
 (segment (start 82 90) (end 82 88) (width 0.6) (layer "B.Cu") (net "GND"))
 (segment (start 116 105) (end 116 98) (width 0.6) (layer "B.Cu") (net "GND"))
 (segment (start 74 22) (end 74 18) (width 1.5) (layer "B.Cu") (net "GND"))
 (segment (start 186.08 121) (end 198 121) (width 1.5) (layer "B.Cu") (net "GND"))
 (segment (start 48.8 68.5) (end 58 68.5) (width 1.5) (layer "B.Cu") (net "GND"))
 (segment (start 74 18) (end 84 18) (width 1.5) (layer "B.Cu") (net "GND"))
 (segment (start 90 88) (end 103.24 83.02) (width 0.6) (layer "B.Cu") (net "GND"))
 (segment (start 90 98) (end 90 88) (width 0.6) (layer "B.Cu") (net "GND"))
 (segment (start 116 98) (end 90 98) (width 0.6) (layer "B.Cu") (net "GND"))
 (segment (start 90 113) (end 90 88) (width 0.6) (layer "B.Cu") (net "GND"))
 (segment (start 87 113) (end 90 113) (width 0.6) (layer "B.Cu") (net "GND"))
 (segment (start 84 18) (end 84 57.62) (width 1.5) (layer "B.Cu") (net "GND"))
 (segment (start 176 42) (end 82 42) (width 1) (layer "F.Cu") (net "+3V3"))
 (segment (start 136 23) (end 136 42) (width 1) (layer "F.Cu") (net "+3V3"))
 (segment (start 172 16) (end 176 16) (width 1) (layer "F.Cu") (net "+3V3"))
 (segment (start 176 16) (end 176 42) (width 1) (layer "F.Cu") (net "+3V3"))
 (segment (start 82 18) (end 69 18) (width 1) (layer "F.Cu") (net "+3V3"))
 (segment (start 82 42) (end 82 18) (width 1) (layer "F.Cu") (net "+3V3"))
 (segment (start 132 23) (end 136 23) (width 1) (layer "F.Cu") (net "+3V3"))
 (segment (start 82 42) (end 82 18) (width 1) (layer "F.Cu") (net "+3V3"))
 (segment (start 136 42) (end 82 42) (width 1) (layer "F.Cu") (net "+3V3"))
 (segment (start 82 18) (end 69 18) (width 1) (layer "F.Cu") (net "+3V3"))
 (segment (start 64 48) (end 64 18) (width 1.5) (layer "B.Cu") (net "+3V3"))
 (segment (start 82 95) (end 82 18) (width 0.6) (layer "B.Cu") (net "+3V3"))
 (segment (start 72 105) (end 68 105) (width 0.6) (layer "B.Cu") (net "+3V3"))
 (segment (start 68 18) (end 69 18) (width 0.6) (layer "B.Cu") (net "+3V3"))
 (segment (start 48.8 48) (end 64 48) (width 1.5) (layer "B.Cu") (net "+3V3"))
 (segment (start 64 18) (end 69 18) (width 1.5) (layer "B.Cu") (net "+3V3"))
 (segment (start 125.62 105) (end 130 105) (width 0.6) (layer "B.Cu") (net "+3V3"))
 (segment (start 82 52.54) (end 103.24 52.54) (width 1.5) (layer "B.Cu") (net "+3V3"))
 (segment (start 69 18) (end 82 18) (width 1.5) (layer "B.Cu") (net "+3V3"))
 (segment (start 82 18) (end 69 18) (width 0.6) (layer "B.Cu") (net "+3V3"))
 (segment (start 68 105) (end 68 18) (width 0.6) (layer "B.Cu") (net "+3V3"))
 (segment (start 130 105) (end 130 95) (width 0.6) (layer "B.Cu") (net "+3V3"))
 (segment (start 82 18) (end 82 52.54) (width 1.5) (layer "B.Cu") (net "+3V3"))
 (segment (start 130 95) (end 82 95) (width 0.6) (layer "B.Cu") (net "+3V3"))
 (segment (start 80 52.54) (end 80 90) (width 0.6) (layer "B.Cu") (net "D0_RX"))
 (segment (start 88 52.54) (end 80 52.54) (width 0.6) (layer "B.Cu") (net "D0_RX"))
 (segment (start 80 90) (end 72 90) (width 0.6) (layer "B.Cu") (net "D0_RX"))
 (segment (start 86 60.16) (end 86 17) (width 0.6) (layer "B.Cu") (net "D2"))
 (segment (start 88 60.16) (end 86 60.16) (width 0.6) (layer "B.Cu") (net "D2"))
 (segment (start 86 17) (end 132 17) (width 0.6) (layer "B.Cu") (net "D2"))
 (segment (start 67 124) (end 67 132) (width 0.6) (layer "B.Cu") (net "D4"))
 (segment (start 88 65.239999) (end 84 65.239999) (width 0.6) (layer "B.Cu") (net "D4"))
 (segment (start 84 124) (end 67 124) (width 0.6) (layer "B.Cu") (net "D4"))
 (segment (start 84 65.239999) (end 84 124) (width 0.6) (layer "B.Cu") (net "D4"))
 (segment (start 88 67.78) (end 82 67.78) (width 0.6) (layer "B.Cu") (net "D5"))
 (segment (start 72.08 124) (end 72.08 132) (width 0.6) (layer "B.Cu") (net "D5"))
 (segment (start 82 67.78) (end 82 124) (width 0.6) (layer "B.Cu") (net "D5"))
 (segment (start 82 124) (end 72.08 124) (width 0.6) (layer "B.Cu") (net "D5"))
 (segment (start 80 124) (end 77.16 124) (width 0.6) (layer "B.Cu") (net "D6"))
 (segment (start 80 70.32) (end 80 124) (width 0.6) (layer "B.Cu") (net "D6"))
 (segment (start 77.16 124) (end 77.16 132) (width 0.6) (layer "B.Cu") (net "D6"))
 (segment (start 88 70.32) (end 80 70.32) (width 0.6) (layer "B.Cu") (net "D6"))
 (segment (start 88 72.86) (end 114 72.86) (width 0.6) (layer "B.Cu") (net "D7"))
 (segment (start 114 30) (end 140 30) (width 0.6) (layer "B.Cu") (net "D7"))
 (segment (start 140 30) (end 147 23.62) (width 0.6) (layer "B.Cu") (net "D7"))
 (segment (start 114 72.86) (end 114 30) (width 0.6) (layer "B.Cu") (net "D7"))
 (segment (start 88 75.4) (end 115 75.4) (width 0.6) (layer "B.Cu") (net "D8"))
 (segment (start 141 32.7) (end 147 26.16) (width 0.6) (layer "B.Cu") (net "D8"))
 (segment (start 115 75.4) (end 115 32.7) (width 0.6) (layer "B.Cu") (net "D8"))
 (segment (start 115 32.7) (end 141 32.7) (width 0.6) (layer "B.Cu") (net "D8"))
 (segment (start 88 77.94) (end 104 77.94) (width 0.6) (layer "B.Cu") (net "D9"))
 (segment (start 104 77.94) (end 104 27) (width 0.6) (layer "B.Cu") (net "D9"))
 (segment (start 104 27) (end 116 27) (width 0.6) (layer "B.Cu") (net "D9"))
 (segment (start 106 25) (end 116 25) (width 0.6) (layer "B.Cu") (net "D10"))
 (segment (start 88 80.48) (end 106 80.48) (width 0.6) (layer "B.Cu") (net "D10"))
 (segment (start 106 80.48) (end 106 25) (width 0.6) (layer "B.Cu") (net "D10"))
 (segment (start 88 83.02) (end 110 85.56) (width 0.6) (layer "B.Cu") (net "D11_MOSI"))
 (segment (start 110 85.56) (end 110 21) (width 0.6) (layer "B.Cu") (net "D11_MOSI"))
 (segment (start 110 21) (end 139 21) (width 0.6) (layer "B.Cu") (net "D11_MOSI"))
 (segment (start 110 21) (end 116 21) (width 0.6) (layer "B.Cu") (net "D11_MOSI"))
 (segment (start 139 18.54) (end 147 18.54) (width 0.6) (layer "B.Cu") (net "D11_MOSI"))
 (segment (start 139 21) (end 139 18.54) (width 0.6) (layer "B.Cu") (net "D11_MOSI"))
 (segment (start 176 19) (end 176 18.54) (width 0.6) (layer "B.Cu") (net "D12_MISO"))
 (segment (start 112 85.56) (end 112 19) (width 0.6) (layer "B.Cu") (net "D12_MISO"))
 (segment (start 176 18.54) (end 172 18.54) (width 0.6) (layer "B.Cu") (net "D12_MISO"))
 (segment (start 112 19) (end 116 19) (width 0.6) (layer "B.Cu") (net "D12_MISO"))
 (segment (start 112 19) (end 176 19) (width 0.6) (layer "B.Cu") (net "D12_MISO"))
 (segment (start 88 85.56) (end 112 85.56) (width 0.6) (layer "B.Cu") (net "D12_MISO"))
 (segment (start 141 23) (end 147 21.08) (width 0.6) (layer "B.Cu") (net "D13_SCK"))
 (segment (start 103.24 50) (end 108 50) (width 0.6) (layer "B.Cu") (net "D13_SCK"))
 (segment (start 108 50) (end 108 23) (width 0.6) (layer "B.Cu") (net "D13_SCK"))
 (segment (start 108 23) (end 116 23) (width 0.6) (layer "B.Cu") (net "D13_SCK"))
 (segment (start 108 23) (end 141 23) (width 0.6) (layer "B.Cu") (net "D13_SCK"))
 (segment (start 77 105) (end 77 113) (width 0.6) (layer "B.Cu") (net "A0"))
 (segment (start 107 105) (end 77 105) (width 0.6) (layer "B.Cu") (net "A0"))
 (segment (start 107 57.62) (end 107 105) (width 0.6) (layer "B.Cu") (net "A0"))
 (segment (start 103.24 57.62) (end 107 57.62) (width 0.6) (layer "B.Cu") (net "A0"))
 (segment (start 120 60.08) (end 183.54 62.62) (width 0.6) (layer "B.Cu") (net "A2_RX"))
 (segment (start 120 62.7) (end 120 60.08) (width 0.6) (layer "B.Cu") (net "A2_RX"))
 (segment (start 103.24 62.7) (end 120 62.7) (width 0.6) (layer "B.Cu") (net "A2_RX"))
 (segment (start 122 62.62) (end 183.54 65.16) (width 0.6) (layer "B.Cu") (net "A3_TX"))
 (segment (start 122 65.239999) (end 122 62.62) (width 0.6) (layer "B.Cu") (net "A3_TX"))
 (segment (start 103.24 65.239999) (end 122 65.239999) (width 0.6) (layer "B.Cu") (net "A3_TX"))
 (segment (start 112 67.78) (end 112 105) (width 0.6) (layer "B.Cu") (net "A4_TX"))
 (segment (start 103.24 67.78) (end 112 67.78) (width 0.6) (layer "B.Cu") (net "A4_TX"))
 (segment (start 112 105) (end 120.54 105) (width 0.6) (layer "B.Cu") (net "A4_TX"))
 (segment (start 114 108) (end 123.08 108) (width 0.6) (layer "B.Cu") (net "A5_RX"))
 (segment (start 123.08 108) (end 123.08 105) (width 0.6) (layer "B.Cu") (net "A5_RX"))
 (segment (start 114 70.32) (end 114 108) (width 0.6) (layer "B.Cu") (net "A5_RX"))
 (segment (start 103.24 70.32) (end 114 70.32) (width 0.6) (layer "B.Cu") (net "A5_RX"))
 (segment (start 195 121) (end 195 57.54) (width 1.5) (layer "B.Cu") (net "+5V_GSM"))
 (segment (start 181 121) (end 195 121) (width 1.5) (layer "B.Cu") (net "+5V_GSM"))
 (segment (start 195 57.54) (end 183.54 55) (width 1.5) (layer "B.Cu") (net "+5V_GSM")))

